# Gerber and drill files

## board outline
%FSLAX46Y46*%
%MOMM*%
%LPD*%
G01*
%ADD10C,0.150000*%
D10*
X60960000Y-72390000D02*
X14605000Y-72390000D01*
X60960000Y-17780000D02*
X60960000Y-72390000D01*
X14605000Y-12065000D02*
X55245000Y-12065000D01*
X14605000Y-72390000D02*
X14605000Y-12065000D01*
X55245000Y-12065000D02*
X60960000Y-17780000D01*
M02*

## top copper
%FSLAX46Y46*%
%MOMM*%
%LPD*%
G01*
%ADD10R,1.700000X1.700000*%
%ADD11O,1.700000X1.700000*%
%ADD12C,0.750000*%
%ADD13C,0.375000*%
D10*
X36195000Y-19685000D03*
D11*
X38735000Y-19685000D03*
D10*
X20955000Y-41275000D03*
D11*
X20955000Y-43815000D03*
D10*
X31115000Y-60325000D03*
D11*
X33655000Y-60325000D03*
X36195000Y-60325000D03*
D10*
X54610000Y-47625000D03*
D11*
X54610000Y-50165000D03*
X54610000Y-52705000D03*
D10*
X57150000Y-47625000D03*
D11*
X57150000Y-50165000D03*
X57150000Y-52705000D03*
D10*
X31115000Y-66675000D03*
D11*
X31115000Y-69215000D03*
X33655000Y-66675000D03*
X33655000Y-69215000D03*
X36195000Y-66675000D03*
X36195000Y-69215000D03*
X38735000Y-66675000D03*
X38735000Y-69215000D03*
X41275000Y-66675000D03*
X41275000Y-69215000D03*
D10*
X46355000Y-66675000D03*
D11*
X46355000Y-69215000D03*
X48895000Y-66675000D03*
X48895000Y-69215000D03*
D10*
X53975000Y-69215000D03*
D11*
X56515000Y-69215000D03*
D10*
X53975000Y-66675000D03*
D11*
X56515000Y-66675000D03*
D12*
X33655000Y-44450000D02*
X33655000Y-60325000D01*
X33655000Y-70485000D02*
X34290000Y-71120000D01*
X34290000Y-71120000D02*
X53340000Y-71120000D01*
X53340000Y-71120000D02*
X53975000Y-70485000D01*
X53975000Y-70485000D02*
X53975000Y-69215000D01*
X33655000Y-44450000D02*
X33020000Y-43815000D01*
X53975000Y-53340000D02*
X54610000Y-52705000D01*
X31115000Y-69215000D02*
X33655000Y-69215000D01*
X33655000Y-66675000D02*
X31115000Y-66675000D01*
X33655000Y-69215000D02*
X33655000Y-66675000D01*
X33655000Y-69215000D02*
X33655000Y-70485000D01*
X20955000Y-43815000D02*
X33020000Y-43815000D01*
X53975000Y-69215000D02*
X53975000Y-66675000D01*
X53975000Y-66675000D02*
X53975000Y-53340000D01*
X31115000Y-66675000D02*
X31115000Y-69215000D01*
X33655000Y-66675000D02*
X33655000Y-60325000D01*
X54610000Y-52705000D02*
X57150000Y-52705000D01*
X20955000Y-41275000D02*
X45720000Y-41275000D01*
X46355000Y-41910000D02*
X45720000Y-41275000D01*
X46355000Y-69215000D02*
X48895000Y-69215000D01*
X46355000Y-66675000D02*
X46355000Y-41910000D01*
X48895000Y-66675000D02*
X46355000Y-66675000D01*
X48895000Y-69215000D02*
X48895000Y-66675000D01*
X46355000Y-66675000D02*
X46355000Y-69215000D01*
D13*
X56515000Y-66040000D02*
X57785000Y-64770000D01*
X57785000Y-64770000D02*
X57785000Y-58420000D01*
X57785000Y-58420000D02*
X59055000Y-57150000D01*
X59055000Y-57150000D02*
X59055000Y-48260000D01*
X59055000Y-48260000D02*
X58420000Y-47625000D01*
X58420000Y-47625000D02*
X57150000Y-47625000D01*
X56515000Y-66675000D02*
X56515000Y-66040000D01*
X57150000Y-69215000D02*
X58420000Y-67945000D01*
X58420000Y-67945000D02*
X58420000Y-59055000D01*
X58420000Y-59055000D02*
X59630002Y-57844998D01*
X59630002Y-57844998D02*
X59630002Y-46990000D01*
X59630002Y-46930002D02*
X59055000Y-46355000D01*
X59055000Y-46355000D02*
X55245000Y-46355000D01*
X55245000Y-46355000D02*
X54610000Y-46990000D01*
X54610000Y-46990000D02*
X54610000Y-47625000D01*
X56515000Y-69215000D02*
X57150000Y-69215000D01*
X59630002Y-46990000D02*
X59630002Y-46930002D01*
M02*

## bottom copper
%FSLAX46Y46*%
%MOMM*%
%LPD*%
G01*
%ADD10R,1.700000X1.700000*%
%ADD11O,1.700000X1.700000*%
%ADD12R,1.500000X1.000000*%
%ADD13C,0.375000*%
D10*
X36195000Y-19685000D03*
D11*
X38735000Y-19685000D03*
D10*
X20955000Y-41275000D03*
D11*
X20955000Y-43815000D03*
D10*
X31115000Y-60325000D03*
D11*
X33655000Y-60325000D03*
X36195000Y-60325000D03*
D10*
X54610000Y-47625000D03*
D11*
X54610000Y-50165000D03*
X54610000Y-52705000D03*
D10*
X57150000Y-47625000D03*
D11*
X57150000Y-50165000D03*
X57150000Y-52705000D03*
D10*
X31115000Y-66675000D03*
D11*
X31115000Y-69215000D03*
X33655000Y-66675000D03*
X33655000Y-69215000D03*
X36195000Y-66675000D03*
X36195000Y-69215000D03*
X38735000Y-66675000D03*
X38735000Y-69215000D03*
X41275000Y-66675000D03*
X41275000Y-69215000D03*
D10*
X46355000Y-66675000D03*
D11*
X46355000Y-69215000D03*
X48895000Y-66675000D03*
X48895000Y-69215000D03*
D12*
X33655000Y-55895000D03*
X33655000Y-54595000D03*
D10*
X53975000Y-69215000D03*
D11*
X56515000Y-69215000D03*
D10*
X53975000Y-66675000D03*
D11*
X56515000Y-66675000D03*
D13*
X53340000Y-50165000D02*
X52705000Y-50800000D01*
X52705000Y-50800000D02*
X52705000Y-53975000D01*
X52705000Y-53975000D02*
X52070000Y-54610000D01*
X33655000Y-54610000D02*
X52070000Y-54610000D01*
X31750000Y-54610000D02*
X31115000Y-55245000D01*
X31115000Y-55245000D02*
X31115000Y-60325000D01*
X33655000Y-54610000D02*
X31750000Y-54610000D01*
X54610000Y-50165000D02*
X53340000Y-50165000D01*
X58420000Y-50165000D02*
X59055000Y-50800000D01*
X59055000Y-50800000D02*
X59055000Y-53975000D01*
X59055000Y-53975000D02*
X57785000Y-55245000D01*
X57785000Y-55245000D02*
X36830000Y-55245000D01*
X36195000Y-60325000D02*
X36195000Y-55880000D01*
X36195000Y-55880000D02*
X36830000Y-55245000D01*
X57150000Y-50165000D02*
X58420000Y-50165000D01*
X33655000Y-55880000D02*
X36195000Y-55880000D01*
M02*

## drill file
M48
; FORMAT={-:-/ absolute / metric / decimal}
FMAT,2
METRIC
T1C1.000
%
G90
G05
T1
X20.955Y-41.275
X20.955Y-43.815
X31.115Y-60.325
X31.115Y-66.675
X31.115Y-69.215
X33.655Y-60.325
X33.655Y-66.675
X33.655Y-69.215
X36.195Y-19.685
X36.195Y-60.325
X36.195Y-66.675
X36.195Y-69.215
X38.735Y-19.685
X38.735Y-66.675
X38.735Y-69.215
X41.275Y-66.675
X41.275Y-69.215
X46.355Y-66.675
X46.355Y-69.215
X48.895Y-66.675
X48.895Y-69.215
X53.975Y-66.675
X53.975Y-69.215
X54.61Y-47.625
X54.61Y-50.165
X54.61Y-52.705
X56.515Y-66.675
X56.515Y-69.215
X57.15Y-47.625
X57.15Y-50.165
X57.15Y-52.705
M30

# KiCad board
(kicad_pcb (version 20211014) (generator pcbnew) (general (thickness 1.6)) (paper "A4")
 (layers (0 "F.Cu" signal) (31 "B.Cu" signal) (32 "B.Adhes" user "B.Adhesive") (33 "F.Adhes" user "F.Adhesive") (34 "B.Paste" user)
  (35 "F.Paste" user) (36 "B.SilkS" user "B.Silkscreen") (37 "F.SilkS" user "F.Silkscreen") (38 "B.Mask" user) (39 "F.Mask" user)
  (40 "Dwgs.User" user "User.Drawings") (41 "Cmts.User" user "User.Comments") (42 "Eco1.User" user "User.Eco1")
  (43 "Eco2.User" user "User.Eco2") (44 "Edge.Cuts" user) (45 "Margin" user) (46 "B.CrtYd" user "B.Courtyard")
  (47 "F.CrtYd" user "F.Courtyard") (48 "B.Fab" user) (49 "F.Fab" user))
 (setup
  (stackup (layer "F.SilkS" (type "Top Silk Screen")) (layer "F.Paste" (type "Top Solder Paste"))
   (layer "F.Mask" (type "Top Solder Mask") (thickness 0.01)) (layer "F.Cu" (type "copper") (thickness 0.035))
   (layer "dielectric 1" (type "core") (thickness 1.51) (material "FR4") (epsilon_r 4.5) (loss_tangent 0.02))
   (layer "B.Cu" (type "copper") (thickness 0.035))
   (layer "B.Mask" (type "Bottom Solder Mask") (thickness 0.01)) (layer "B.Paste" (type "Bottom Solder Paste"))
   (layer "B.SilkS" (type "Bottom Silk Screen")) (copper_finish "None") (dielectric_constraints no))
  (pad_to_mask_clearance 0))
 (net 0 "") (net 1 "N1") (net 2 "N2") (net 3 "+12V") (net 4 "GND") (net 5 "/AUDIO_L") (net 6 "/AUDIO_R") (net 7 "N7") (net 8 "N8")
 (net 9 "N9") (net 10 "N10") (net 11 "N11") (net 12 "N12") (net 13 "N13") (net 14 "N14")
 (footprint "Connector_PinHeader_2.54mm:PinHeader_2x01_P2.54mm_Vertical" (layer "F.Cu") (at 36.195 19.685)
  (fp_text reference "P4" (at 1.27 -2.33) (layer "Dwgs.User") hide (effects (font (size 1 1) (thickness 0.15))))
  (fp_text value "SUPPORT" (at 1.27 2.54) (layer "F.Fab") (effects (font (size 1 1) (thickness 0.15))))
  (pad "1" thru_hole rect (at 0 0) (size 1.7 1.7) (drill 1) (layers *.Cu *.Mask) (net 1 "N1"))
  (pad "2" thru_hole oval (at 2.54 0) (size 1.7 1.7) (drill 1) (layers *.Cu *.Mask) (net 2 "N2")))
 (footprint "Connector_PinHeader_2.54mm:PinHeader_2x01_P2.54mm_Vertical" (layer "F.Cu") (at 20.955 41.275 -90)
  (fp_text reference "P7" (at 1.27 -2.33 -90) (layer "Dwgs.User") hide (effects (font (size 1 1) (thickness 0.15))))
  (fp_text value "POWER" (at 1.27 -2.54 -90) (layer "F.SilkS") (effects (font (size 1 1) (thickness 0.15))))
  (pad "1" thru_hole rect (at 0 0 270) (size 1.7 1.7) (drill 1) (layers *.Cu *.Mask) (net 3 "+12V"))
  (pad "2" thru_hole oval (at 2.54 0 270) (size 1.7 1.7) (drill 1) (layers *.Cu *.Mask) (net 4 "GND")))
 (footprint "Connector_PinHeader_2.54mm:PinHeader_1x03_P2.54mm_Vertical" (layer "F.Cu") (at 31.115 60.325 90)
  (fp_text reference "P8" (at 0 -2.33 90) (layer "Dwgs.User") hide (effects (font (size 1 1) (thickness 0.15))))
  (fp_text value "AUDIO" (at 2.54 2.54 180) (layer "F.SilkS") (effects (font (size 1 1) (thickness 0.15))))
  (pad "1" thru_hole rect (at 0 0 90) (size 1.7 1.7) (drill 1) (layers *.Cu *.Mask) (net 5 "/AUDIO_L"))
  (pad "2" thru_hole oval (at 0 2.54 90) (size 1.7 1.7) (drill 1) (layers *.Cu *.Mask) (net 4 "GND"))
  (pad "3" thru_hole oval (at 0 5.08 90) (size 1.7 1.7) (drill 1) (layers *.Cu *.Mask) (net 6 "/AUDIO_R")))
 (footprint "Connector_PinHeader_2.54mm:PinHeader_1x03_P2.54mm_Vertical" (layer "F.Cu") (at 54.61 47.625)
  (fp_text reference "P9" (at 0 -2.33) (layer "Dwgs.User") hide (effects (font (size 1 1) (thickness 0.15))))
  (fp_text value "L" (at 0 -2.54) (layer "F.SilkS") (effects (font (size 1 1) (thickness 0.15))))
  (pad "1" thru_hole rect (at 0 0) (size 1.7 1.7) (drill 1) (layers *.Cu *.Mask) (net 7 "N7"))
  (pad "2" thru_hole oval (at 0 2.54) (size 1.7 1.7) (drill 1) (layers *.Cu *.Mask) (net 5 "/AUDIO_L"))
  (pad "3" thru_hole oval (at 0 5.08) (size 1.7 1.7) (drill 1) (layers *.Cu *.Mask) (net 4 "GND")))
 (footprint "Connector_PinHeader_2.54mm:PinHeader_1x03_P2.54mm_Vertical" (layer "F.Cu") (at 57.15 47.625)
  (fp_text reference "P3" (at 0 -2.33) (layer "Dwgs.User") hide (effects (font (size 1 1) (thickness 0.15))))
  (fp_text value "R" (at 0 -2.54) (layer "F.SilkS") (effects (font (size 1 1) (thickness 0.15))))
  (pad "1" thru_hole rect (at 0 0) (size 1.7 1.7) (drill 1) (layers *.Cu *.Mask) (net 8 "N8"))
  (pad "2" thru_hole oval (at 0 2.54) (size 1.7 1.7) (drill 1) (layers *.Cu *.Mask) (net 6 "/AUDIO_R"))
  (pad "3" thru_hole oval (at 0 5.08) (size 1.7 1.7) (drill 1) (layers *.Cu *.Mask) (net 4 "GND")))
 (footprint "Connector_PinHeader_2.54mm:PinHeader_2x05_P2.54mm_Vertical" (layer "B.Cu") (at 31.115 66.675 -90)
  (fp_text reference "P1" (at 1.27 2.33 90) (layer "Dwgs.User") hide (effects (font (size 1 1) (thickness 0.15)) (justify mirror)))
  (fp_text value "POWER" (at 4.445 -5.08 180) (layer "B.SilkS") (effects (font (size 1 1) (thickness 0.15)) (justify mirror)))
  (pad "1" thru_hole rect (at 0 0 270) (size 1.7 1.7) (drill 1) (layers *.Cu *.Mask) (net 4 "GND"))
  (pad "2" thru_hole oval (at 2.54 0 270) (size 1.7 1.7) (drill 1) (layers *.Cu *.Mask) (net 4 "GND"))
  (pad "3" thru_hole oval (at 0 -2.54 270) (size 1.7 1.7) (drill 1) (layers *.Cu *.Mask) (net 4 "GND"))
  (pad "4" thru_hole oval (at 2.54 -2.54 270) (size 1.7 1.7) (drill 1) (layers *.Cu *.Mask) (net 4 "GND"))
  (pad "5" thru_hole oval (at 0 -5.08 270) (size 1.7 1.7) (drill 1) (layers *.Cu *.Mask) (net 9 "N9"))
  (pad "6" thru_hole oval (at 2.54 -5.08 270) (size 1.7 1.7) (drill 1) (layers *.Cu *.Mask) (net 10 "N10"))
  (pad "7" thru_hole oval (at 0 -7.62 270) (size 1.7 1.7) (drill 1) (layers *.Cu *.Mask) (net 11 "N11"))
  (pad "8" thru_hole oval (at 2.54 -7.62 270) (size 1.7 1.7) (drill 1) (layers *.Cu *.Mask) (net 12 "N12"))
  (pad "9" thru_hole oval (at 0 -10.16 270) (size 1.7 1.7) (drill 1) (layers *.Cu *.Mask) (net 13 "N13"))
  (pad "10" thru_hole oval (at 2.54 -10.16 270) (size 1.7 1.7) (drill 1) (layers *.Cu *.Mask) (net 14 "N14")))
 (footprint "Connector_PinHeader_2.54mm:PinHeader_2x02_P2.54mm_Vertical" (layer "B.Cu") (at 46.355 66.675 -90)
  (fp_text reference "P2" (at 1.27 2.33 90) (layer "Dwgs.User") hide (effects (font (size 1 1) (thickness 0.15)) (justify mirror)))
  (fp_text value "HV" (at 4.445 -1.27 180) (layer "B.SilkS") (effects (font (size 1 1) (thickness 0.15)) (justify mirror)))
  (pad "1" thru_hole rect (at 0 0 270) (size 1.7 1.7) (drill 1) (layers *.Cu *.Mask) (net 3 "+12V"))
  (pad "2" thru_hole oval (at 2.54 0 270) (size 1.7 1.7) (drill 1) (layers *.Cu *.Mask) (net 3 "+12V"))
  (pad "3" thru_hole oval (at 0 -2.54 270) (size 1.7 1.7) (drill 1) (layers *.Cu *.Mask) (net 3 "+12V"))
  (pad "4" thru_hole oval (at 2.54 -2.54 270) (size 1.7 1.7) (drill 1) (layers *.Cu *.Mask) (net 3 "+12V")))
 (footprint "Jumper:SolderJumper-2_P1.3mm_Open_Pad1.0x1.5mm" (layer "B.Cu") (at 33.655 55.245 90)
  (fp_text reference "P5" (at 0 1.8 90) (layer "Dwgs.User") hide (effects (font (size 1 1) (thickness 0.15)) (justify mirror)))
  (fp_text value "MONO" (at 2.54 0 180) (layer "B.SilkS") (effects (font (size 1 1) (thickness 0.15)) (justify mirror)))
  (pad "1" smd rect (at -0.65 0 90) (size 1 1.5) (layers "B.Cu" "B.Mask") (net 6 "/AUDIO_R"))
  (pad "2" smd rect (at 0.65 0 90) (size 1 1.5) (layers "B.Cu" "B.Mask") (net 5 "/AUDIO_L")))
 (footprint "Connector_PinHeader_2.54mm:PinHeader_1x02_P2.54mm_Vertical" (layer "B.Cu") (at 53.975 69.215 -90)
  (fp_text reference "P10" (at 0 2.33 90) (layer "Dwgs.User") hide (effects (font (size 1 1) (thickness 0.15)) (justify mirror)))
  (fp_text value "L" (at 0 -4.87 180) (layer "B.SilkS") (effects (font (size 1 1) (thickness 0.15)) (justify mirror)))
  (pad "1" thru_hole rect (at 0 0 270) (size 1.7 1.7) (drill 1) (layers *.Cu *.Mask) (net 4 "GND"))
  (pad "2" thru_hole oval (at 0 -2.54 270) (size 1.7 1.7) (drill 1) (layers *.Cu *.Mask) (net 7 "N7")))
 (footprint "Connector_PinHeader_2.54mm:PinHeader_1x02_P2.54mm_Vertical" (layer "B.Cu") (at 53.975 66.675 -90)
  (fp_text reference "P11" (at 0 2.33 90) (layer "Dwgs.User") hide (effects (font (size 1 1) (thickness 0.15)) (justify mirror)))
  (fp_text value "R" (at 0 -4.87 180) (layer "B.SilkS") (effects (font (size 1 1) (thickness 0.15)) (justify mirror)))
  (pad "1" thru_hole rect (at 0 0 270) (size 1.7 1.7) (drill 1) (layers *.Cu *.Mask) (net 4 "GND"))
  (pad "2" thru_hole oval (at 0 -2.54 270) (size 1.7 1.7) (drill 1) (layers *.Cu *.Mask) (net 8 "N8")))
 (gr_line (start 60.96 72.39) (end 14.605 72.39) (layer "Edge.Cuts") (width 0.15))
 (gr_line (start 60.96 17.78) (end 60.96 72.39) (layer "Edge.Cuts") (width 0.15))
 (gr_line (start 14.605 12.065) (end 55.245 12.065) (layer "Edge.Cuts") (width 0.15))
 (gr_line (start 14.605 72.39) (end 14.605 12.065) (layer "Edge.Cuts") (width 0.15))
 (gr_line (start 55.245 12.065) (end 60.96 17.78) (layer "Edge.Cuts") (width 0.15))
 (segment (start 33.655 44.45) (end 33.655 60.325) (width 0.75) (layer "F.Cu") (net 4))
 (segment (start 33.655 70.485) (end 34.29 71.12) (width 0.75) (layer "F.Cu") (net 4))
 (segment (start 34.29 71.12) (end 53.34 71.12) (width 0.75) (layer "F.Cu") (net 4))
 (segment (start 53.34 71.12) (end 53.975 70.485) (width 0.75) (layer "F.Cu") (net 4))
 (segment (start 53.975 70.485) (end 53.975 69.215) (width 0.75) (layer "F.Cu") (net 4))
 (segment (start 33.655 44.45) (end 33.02 43.815) (width 0.75) (layer "F.Cu") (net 4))
 (segment (start 53.975 53.34) (end 54.61 52.705) (width 0.75) (layer "F.Cu") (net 4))
 (segment (start 31.115 69.215) (end 33.655 69.215) (width 0.75) (layer "F.Cu") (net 4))
 (segment (start 33.655 66.675) (end 31.115 66.675) (width 0.75) (layer "F.Cu") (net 4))
 (segment (start 33.655 69.215) (end 33.655 66.675) (width 0.75) (layer "F.Cu") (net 4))
 (segment (start 33.655 69.215) (end 33.655 70.485) (width 0.75) (layer "F.Cu") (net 4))
 (segment (start 20.955 43.815) (end 33.02 43.815) (width 0.75) (layer "F.Cu") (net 4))
 (segment (start 53.975 69.215) (end 53.975 66.675) (width 0.75) (layer "F.Cu") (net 4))
 (segment (start 53.975 66.675) (end 53.975 53.34) (width 0.75) (layer "F.Cu") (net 4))
 (segment (start 31.115 66.675) (end 31.115 69.215) (width 0.75) (layer "F.Cu") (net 4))
 (segment (start 33.655 66.675) (end 33.655 60.325) (width 0.75) (layer "F.Cu") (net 4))
 (segment (start 54.61 52.705) (end 57.15 52.705) (width 0.75) (layer "F.Cu") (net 4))
 (segment (start 20.955 41.275) (end 45.72 41.275) (width 0.75) (layer "F.Cu") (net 3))
 (segment (start 46.355 41.91) (end 45.72 41.275) (width 0.75) (layer "F.Cu") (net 3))
 (segment (start 46.355 69.215) (end 48.895 69.215) (width 0.75) (layer "F.Cu") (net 3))
 (segment (start 46.355 66.675) (end 46.355 41.91) (width 0.75) (layer "F.Cu") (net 3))
 (segment (start 48.895 66.675) (end 46.355 66.675) (width 0.75) (layer "F.Cu") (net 3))
 (segment (start 48.895 69.215) (end 48.895 66.675) (width 0.75) (layer "F.Cu") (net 3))
 (segment (start 46.355 66.675) (end 46.355 69.215) (width 0.75) (layer "F.Cu") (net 3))
 (segment (start 56.515 66.04) (end 57.785 64.77) (width 0.375) (layer "F.Cu") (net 8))
 (segment (start 57.785 64.77) (end 57.785 58.42) (width 0.375) (layer "F.Cu") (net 8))
 (segment (start 57.785 58.42) (end 59.055 57.15) (width 0.375) (layer "F.Cu") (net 8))
 (segment (start 59.055 57.15) (end 59.055 48.26) (width 0.375) (layer "F.Cu") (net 8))
 (segment (start 59.055 48.26) (end 58.42 47.625) (width 0.375) (layer "F.Cu") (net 8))
 (segment (start 58.42 47.625) (end 57.15 47.625) (width 0.375) (layer "F.Cu") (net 8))
 (segment (start 56.515 66.675) (end 56.515 66.04) (width 0.375) (layer "F.Cu") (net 8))
 (segment (start 53.34 50.165) (end 52.705 50.8) (width 0.375) (layer "B.Cu") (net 5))
 (segment (start 52.705 50.8) (end 52.705 53.975) (width 0.375) (layer "B.Cu") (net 5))
 (segment (start 52.705 53.975) (end 52.07 54.61) (width 0.375) (layer "B.Cu") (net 5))
 (segment (start 33.655 54.61) (end 52.07 54.61) (width 0.375) (layer "B.Cu") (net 5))
 (segment (start 31.75 54.61) (end 31.115 55.245) (width 0.375) (layer "B.Cu") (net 5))
 (segment (start 31.115 55.245) (end 31.115 60.325) (width 0.375) (layer "B.Cu") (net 5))
 (segment (start 33.655 54.61) (end 31.75 54.61) (width 0.375) (layer "B.Cu") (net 5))
 (segment (start 54.61 50.165) (end 53.34 50.165) (width 0.375) (layer "B.Cu") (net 5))
 (segment (start 58.42 50.165) (end 59.055 50.8) (width 0.375) (layer "B.Cu") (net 6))
 (segment (start 59.055 50.8) (end 59.055 53.975) (width 0.375) (layer "B.Cu") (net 6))
 (segment (start 59.055 53.975) (end 57.785 55.245) (width 0.375) (layer "B.Cu") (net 6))
 (segment (start 57.785 55.245) (end 36.83 55.245) (width 0.375) (layer "B.Cu") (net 6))
 (segment (start 36.195 60.325) (end 36.195 55.88) (width 0.375) (layer "B.Cu") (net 6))
 (segment (start 36.195 55.88) (end 36.83 55.245) (width 0.375) (layer "B.Cu") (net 6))
 (segment (start 57.15 50.165) (end 58.42 50.165) (width 0.375) (layer "B.Cu") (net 6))
 (segment (start 33.655 55.88) (end 36.195 55.88) (width 0.375) (layer "B.Cu") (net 6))
 (segment (start 57.15 69.215) (end 58.42 67.945) (width 0.375) (layer "F.Cu") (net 7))
 (segment (start 58.42 67.945) (end 58.42 59.055) (width 0.375) (layer "F.Cu") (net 7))
 (segment (start 58.42 59.055) (end 59.630002 57.844998) (width 0.375) (layer "F.Cu") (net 7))
 (segment (start 59.630002 57.844998) (end 59.630002 46.99) (width 0.375) (layer "F.Cu") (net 7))
 (segment (start 59.630002 46.930002) (end 59.055 46.355) (width 0.375) (layer "F.Cu") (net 7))
 (segment (start 59.055 46.355) (end 55.245 46.355) (width 0.375) (layer "F.Cu") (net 7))
 (segment (start 55.245 46.355) (end 54.61 46.99) (width 0.375) (layer "F.Cu") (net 7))
 (segment (start 54.61 46.99) (end 54.61 47.625) (width 0.375) (layer "F.Cu") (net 7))
 (segment (start 56.515 69.215) (end 57.15 69.215) (width 0.375) (layer "F.Cu") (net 7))
 (segment (start 59.630002 46.99) (end 59.630002 46.930002) (width 0.375) (layer "F.Cu") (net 7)))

